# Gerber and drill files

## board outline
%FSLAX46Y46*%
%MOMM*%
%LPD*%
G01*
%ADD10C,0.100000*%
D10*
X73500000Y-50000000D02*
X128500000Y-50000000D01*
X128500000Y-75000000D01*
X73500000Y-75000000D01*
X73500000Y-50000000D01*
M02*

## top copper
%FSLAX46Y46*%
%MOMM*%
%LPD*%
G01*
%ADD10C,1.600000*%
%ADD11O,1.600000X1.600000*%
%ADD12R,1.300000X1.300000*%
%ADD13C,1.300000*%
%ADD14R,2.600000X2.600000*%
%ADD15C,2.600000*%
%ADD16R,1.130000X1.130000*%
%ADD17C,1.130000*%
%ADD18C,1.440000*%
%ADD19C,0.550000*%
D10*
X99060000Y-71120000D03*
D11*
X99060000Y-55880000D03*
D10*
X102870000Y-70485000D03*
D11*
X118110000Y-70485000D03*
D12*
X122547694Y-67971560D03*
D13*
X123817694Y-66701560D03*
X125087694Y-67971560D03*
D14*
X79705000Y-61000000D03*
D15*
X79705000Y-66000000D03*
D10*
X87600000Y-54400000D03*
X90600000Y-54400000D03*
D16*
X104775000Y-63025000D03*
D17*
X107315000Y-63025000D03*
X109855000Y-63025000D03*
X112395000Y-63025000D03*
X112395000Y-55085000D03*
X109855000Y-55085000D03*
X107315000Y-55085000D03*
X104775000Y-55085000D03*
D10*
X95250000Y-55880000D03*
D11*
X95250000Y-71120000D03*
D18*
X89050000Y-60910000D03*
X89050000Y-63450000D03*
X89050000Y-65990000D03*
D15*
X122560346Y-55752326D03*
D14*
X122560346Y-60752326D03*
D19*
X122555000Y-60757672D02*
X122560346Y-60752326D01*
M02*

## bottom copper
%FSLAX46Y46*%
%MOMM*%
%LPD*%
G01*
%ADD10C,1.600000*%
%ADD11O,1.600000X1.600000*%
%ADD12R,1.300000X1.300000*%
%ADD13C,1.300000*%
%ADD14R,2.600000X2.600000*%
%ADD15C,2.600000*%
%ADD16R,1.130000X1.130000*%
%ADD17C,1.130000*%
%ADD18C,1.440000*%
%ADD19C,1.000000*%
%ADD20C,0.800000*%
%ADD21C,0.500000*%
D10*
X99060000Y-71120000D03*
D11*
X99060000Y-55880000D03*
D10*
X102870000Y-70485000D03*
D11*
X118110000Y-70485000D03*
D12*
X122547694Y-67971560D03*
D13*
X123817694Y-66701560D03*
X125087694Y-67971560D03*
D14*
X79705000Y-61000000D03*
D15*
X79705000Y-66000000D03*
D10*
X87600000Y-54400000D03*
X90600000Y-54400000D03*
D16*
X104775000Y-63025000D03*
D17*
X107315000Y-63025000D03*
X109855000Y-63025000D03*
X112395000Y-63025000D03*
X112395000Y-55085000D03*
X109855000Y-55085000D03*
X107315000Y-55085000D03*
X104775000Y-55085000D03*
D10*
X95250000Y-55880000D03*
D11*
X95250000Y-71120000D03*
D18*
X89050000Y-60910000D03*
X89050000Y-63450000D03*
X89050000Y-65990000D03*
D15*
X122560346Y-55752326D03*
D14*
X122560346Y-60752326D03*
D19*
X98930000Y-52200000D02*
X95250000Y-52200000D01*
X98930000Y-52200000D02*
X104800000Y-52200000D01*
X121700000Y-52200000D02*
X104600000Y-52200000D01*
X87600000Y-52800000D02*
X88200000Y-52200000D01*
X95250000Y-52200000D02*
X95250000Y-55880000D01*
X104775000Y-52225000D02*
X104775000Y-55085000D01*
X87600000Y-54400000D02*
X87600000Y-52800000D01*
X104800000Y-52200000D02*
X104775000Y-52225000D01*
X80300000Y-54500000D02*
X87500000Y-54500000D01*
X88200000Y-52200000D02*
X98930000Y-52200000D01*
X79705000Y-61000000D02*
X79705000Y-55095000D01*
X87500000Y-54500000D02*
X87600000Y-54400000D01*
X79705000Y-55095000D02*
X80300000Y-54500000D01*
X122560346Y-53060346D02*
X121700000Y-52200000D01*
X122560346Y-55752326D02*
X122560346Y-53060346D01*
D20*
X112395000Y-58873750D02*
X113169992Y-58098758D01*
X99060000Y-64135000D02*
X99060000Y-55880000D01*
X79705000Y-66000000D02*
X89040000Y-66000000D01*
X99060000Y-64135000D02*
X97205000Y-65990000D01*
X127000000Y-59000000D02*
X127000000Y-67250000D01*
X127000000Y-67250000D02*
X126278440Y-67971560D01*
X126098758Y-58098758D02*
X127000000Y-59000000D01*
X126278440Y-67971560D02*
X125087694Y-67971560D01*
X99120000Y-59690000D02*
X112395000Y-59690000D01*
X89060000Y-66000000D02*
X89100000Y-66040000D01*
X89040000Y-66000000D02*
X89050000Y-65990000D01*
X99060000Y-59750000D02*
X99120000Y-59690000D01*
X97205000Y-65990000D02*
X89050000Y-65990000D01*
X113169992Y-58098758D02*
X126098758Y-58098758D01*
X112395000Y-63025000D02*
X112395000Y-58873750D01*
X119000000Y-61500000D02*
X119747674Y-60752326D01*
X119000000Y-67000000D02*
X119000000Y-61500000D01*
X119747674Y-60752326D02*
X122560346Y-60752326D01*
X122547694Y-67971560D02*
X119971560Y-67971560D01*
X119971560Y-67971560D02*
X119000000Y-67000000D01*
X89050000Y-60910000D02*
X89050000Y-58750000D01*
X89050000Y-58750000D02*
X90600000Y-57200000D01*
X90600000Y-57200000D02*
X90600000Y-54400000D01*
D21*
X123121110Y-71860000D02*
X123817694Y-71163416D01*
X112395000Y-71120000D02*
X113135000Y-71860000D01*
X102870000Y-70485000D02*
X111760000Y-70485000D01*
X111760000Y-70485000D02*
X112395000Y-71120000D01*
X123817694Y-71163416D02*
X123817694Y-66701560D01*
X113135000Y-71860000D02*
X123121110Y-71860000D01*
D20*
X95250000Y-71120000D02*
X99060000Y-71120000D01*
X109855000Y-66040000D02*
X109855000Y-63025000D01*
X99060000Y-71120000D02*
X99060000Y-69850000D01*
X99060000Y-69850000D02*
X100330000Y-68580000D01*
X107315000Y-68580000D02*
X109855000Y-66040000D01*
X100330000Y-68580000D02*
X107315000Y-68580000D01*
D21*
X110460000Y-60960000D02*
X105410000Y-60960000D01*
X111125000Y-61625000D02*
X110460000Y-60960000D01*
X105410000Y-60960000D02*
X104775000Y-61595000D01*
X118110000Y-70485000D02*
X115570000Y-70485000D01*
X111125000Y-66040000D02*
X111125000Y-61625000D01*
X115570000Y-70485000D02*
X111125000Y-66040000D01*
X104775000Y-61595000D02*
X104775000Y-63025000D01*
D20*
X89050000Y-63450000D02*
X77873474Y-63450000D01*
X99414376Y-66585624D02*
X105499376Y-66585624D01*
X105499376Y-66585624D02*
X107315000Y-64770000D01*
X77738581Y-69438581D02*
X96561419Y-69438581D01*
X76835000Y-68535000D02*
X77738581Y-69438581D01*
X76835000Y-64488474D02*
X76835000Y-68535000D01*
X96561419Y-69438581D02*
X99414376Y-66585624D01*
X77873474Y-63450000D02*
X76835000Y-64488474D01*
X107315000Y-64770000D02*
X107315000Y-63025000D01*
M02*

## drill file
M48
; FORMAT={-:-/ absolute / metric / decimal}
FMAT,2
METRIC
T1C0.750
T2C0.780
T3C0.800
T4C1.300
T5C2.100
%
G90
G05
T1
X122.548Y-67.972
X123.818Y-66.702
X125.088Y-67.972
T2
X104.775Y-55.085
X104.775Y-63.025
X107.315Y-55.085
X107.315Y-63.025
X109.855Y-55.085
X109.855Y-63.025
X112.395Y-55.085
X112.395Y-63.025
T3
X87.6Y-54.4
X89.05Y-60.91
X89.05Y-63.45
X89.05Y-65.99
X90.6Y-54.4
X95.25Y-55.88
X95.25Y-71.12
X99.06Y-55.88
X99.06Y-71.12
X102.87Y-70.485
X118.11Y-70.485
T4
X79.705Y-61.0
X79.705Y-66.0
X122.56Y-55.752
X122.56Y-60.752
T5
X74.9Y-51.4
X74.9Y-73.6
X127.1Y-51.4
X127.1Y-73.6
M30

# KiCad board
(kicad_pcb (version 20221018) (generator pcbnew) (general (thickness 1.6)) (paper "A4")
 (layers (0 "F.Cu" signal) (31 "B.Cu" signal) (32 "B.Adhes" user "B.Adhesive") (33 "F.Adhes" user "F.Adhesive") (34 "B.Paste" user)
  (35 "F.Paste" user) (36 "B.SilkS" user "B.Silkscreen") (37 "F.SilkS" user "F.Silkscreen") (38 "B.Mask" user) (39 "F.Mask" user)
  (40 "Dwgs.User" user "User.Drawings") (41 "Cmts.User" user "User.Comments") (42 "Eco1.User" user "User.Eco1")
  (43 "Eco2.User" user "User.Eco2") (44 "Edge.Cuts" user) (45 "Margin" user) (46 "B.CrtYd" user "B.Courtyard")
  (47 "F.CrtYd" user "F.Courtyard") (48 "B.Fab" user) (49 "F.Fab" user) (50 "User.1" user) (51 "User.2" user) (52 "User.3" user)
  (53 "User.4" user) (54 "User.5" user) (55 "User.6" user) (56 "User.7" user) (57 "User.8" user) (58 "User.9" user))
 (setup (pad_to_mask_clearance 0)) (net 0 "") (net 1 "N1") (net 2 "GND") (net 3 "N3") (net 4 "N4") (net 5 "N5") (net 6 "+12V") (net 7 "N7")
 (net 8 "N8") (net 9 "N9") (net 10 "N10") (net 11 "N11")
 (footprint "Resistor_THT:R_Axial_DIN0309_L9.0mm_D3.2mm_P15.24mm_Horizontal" (layer "F.Cu") (at 99.06 71.12 90)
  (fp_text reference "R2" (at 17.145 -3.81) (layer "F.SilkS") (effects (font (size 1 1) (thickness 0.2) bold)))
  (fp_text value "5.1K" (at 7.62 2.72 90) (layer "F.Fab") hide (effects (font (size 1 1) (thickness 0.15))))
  (pad "1" thru_hole circle (at 0 0 90) (size 1.6 1.6) (drill 0.8) (layers "*.Cu" "*.Mask") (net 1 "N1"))
  (pad "2" thru_hole oval (at 15.24 0 90) (size 1.6 1.6) (drill 0.8) (layers "*.Cu" "*.Mask") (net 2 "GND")))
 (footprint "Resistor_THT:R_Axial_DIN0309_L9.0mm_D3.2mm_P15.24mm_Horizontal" (layer "F.Cu") (at 102.87 70.485)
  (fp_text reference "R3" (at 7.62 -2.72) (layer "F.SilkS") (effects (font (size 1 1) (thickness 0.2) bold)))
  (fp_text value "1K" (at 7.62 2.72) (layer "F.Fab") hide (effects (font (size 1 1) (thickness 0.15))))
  (pad "1" thru_hole circle (at 0 0) (size 1.6 1.6) (drill 0.8) (layers "*.Cu" "*.Mask") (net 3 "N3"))
  (pad "2" thru_hole oval (at 15.24 0) (size 1.6 1.6) (drill 0.8) (layers "*.Cu" "*.Mask") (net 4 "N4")))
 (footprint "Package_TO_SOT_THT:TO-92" (layer "F.Cu") (at 122.547694 67.97156)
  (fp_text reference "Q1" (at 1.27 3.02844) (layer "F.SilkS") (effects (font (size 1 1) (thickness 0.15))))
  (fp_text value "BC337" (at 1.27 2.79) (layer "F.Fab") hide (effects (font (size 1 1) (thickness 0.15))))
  (pad "1" thru_hole rect (at 0 0) (size 1.3 1.3) (drill 0.75) (layers "*.Cu" "*.Mask") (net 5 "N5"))
  (pad "2" thru_hole circle (at 1.27 -1.27) (size 1.3 1.3) (drill 0.75) (layers "*.Cu" "*.Mask") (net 3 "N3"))
  (pad "3" thru_hole circle (at 2.54 0) (size 1.3 1.3) (drill 0.75) (layers "*.Cu" "*.Mask") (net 2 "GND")))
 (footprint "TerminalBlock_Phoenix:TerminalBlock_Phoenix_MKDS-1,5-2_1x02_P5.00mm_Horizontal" (layer "F.Cu") (at 79.705 61 -90)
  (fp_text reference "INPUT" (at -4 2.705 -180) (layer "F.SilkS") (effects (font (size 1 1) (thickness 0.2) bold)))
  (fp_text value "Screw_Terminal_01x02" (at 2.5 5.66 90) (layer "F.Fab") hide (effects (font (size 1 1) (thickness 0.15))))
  (pad "1" thru_hole rect (at 0 0 270) (size 2.6 2.6) (drill 1.3) (layers "*.Cu" "*.Mask") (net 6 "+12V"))
  (pad "2" thru_hole circle (at 5 0 270) (size 2.6 2.6) (drill 1.3) (layers "*.Cu" "*.Mask") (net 2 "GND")))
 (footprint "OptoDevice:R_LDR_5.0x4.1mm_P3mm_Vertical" (layer "F.Cu") (at 87.6 54.4)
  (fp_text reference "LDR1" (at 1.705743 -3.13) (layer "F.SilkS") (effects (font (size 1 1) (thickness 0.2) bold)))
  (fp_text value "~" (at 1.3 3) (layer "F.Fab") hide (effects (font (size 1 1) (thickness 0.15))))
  (pad "1" thru_hole circle (at 0 0) (size 1.6 1.6) (drill 0.8) (layers "*.Cu" "*.Mask") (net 6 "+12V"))
  (pad "2" thru_hole circle (at 3 0) (size 1.6 1.6) (drill 0.8) (layers "*.Cu" "*.Mask") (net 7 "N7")))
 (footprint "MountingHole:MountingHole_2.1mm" (layer "F.Cu") (at 74.9 51.4)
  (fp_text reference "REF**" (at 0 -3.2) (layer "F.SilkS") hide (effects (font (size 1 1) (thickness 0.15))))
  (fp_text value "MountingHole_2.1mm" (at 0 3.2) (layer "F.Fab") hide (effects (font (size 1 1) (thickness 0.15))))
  (pad "" np_thru_hole circle (at 0 0) (size 2.1 2.1) (drill 2.1) (layers "F&B.Cu" "*.Mask")))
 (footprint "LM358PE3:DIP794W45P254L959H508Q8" (layer "F.Cu") (at 108.585 59.055 90)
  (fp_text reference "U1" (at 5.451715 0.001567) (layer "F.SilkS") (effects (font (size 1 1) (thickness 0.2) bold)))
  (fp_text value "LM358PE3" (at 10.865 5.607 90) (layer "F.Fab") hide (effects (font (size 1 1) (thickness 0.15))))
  (pad "1" thru_hole rect (at -3.97 -3.81 90) (size 1.13 1.13) (drill 0.78) (layers "*.Cu" "*.Mask") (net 4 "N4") (solder_mask_margin 0.102))
  (pad "2" thru_hole circle (at -3.97 -1.27 90) (size 1.13 1.13) (drill 0.78) (layers "*.Cu" "*.Mask") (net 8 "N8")
   (solder_mask_margin 0.102))
  (pad "3" thru_hole circle (at -3.97 1.27 90) (size 1.13 1.13) (drill 0.78) (layers "*.Cu" "*.Mask") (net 1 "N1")
   (solder_mask_margin 0.102))
  (pad "4" thru_hole circle (at -3.97 3.81 90) (size 1.13 1.13) (drill 0.78) (layers "*.Cu" "*.Mask") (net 2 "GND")
   (solder_mask_margin 0.102))
  (pad "5" thru_hole circle (at 3.97 3.81 90) (size 1.13 1.13) (drill 0.78) (layers "*.Cu" "*.Mask") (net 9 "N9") (solder_mask_margin 0.102))
  (pad "6" thru_hole circle (at 3.97 1.27 90) (size 1.13 1.13) (drill 0.78) (layers "*.Cu" "*.Mask") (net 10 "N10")
   (solder_mask_margin 0.102))
  (pad "7" thru_hole circle (at 3.97 -1.27 90) (size 1.13 1.13) (drill 0.78) (layers "*.Cu" "*.Mask") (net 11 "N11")
   (solder_mask_margin 0.102))
  (pad "8" thru_hole circle (at 3.97 -3.81 90) (size 1.13 1.13) (drill 0.78) (layers "*.Cu" "*.Mask") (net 6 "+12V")
   (solder_mask_margin 0.102)))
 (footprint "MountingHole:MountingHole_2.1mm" (layer "F.Cu") (at 74.9 73.6)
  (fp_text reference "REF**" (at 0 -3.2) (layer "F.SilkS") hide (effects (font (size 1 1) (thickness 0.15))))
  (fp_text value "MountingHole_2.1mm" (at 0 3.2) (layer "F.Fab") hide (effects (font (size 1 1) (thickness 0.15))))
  (pad "" np_thru_hole circle (at 0 0) (size 2.1 2.1) (drill 2.1) (layers "F&B.Cu" "*.Mask")))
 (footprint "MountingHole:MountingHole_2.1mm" (layer "F.Cu") (at 127.1 51.4)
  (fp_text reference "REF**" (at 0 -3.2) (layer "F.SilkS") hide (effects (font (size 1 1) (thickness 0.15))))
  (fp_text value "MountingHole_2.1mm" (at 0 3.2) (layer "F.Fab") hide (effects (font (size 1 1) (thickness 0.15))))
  (pad "" np_thru_hole circle (at 0 0) (size 2.1 2.1) (drill 2.1) (layers "F&B.Cu" "*.Mask")))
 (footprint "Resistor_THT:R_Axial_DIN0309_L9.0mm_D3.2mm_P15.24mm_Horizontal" (layer "F.Cu") (at 95.25 55.88 -90)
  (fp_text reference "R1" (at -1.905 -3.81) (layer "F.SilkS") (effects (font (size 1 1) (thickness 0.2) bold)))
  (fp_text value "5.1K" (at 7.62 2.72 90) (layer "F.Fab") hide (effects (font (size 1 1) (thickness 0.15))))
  (pad "1" thru_hole circle (at 0 0 270) (size 1.6 1.6) (drill 0.8) (layers "*.Cu" "*.Mask") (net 6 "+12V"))
  (pad "2" thru_hole oval (at 15.24 0 270) (size 1.6 1.6) (drill 0.8) (layers "*.Cu" "*.Mask") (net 1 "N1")))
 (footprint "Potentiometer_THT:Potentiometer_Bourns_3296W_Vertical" (layer "F.Cu") (at 89.05 60.91 90)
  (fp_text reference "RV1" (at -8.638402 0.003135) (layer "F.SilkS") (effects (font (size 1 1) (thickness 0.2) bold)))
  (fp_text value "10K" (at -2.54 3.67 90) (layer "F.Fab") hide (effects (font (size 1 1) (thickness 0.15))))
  (pad "1" thru_hole circle (at 0 0 90) (size 1.44 1.44) (drill 0.8) (layers "*.Cu" "*.Mask") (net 7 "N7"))
  (pad "2" thru_hole circle (at -2.54 0 90) (size 1.44 1.44) (drill 0.8) (layers "*.Cu" "*.Mask") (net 8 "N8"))
  (pad "3" thru_hole circle (at -5.08 0 90) (size 1.44 1.44) (drill 0.8) (layers "*.Cu" "*.Mask") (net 2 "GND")))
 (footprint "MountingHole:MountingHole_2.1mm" (layer "F.Cu") (at 127.1 73.6)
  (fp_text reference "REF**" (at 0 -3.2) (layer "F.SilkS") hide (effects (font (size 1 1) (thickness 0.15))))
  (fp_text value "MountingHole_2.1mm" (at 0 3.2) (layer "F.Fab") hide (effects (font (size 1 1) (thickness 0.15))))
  (pad "" np_thru_hole circle (at 0 0) (size 2.1 2.1) (drill 2.1) (layers "*.Cu" "*.Mask")))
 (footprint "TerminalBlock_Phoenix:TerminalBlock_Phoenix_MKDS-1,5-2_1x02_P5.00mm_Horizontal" (layer "F.Cu") (at 122.560346 60.752326 90)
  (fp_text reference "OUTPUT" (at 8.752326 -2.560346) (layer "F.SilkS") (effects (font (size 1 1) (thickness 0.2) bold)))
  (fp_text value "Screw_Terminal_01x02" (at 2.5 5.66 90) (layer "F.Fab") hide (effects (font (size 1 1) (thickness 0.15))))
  (pad "1" thru_hole circle (at 5 0 90) (size 2.6 2.6) (drill 1.3) (layers "*.Cu" "*.Mask") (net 6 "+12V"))
  (pad "2" thru_hole rect (at 0 0 90) (size 2.6 2.6) (drill 1.3) (layers "*.Cu" "*.Mask") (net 5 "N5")))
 (gr_rect (start 73.5 50) (end 128.5 75) (stroke (width 0.1) (type default)) (fill none) (layer "Edge.Cuts"))
 (segment (start 98.93 52.2) (end 95.25 52.2) (width 1) (layer "B.Cu") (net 6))
 (segment (start 98.93 52.2) (end 104.8 52.2) (width 1) (layer "B.Cu") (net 6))
 (segment (start 121.7 52.2) (end 104.6 52.2) (width 1) (layer "B.Cu") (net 6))
 (segment (start 87.6 52.8) (end 88.2 52.2) (width 1) (layer "B.Cu") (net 6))
 (segment (start 95.25 52.2) (end 95.25 55.88) (width 1) (layer "B.Cu") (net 6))
 (segment (start 104.775 52.225) (end 104.775 55.085) (width 1) (layer "B.Cu") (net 6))
 (segment (start 87.6 54.4) (end 87.6 52.8) (width 1) (layer "B.Cu") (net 6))
 (segment (start 104.8 52.2) (end 104.775 52.225) (width 1) (layer "B.Cu") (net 6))
 (segment (start 80.3 54.5) (end 87.5 54.5) (width 1) (layer "B.Cu") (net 6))
 (segment (start 88.2 52.2) (end 98.93 52.2) (width 1) (layer "B.Cu") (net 6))
 (segment (start 79.705 61) (end 79.705 55.095) (width 1) (layer "B.Cu") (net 6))
 (segment (start 87.5 54.5) (end 87.6 54.4) (width 1) (layer "B.Cu") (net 6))
 (segment (start 79.705 55.095) (end 80.3 54.5) (width 1) (layer "B.Cu") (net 6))
 (segment (start 122.560346 53.060346) (end 121.7 52.2) (width 1) (layer "B.Cu") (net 6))
 (segment (start 122.560346 55.752326) (end 122.560346 53.060346) (width 1) (layer "B.Cu") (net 6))
 (segment (start 112.395 58.87375) (end 113.169992 58.098758) (width 0.8) (layer "B.Cu") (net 2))
 (segment (start 99.06 64.135) (end 99.06 55.88) (width 0.8) (layer "B.Cu") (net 2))
 (segment (start 79.705 66) (end 89.04 66) (width 0.8) (layer "B.Cu") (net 2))
 (segment (start 99.06 64.135) (end 97.205 65.99) (width 0.8) (layer "B.Cu") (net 2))
 (segment (start 127 59) (end 127 67.25) (width 0.8) (layer "B.Cu") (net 2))
 (segment (start 127 67.25) (end 126.27844 67.97156) (width 0.8) (layer "B.Cu") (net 2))
 (segment (start 126.098758 58.098758) (end 127 59) (width 0.8) (layer "B.Cu") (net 2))
 (segment (start 126.27844 67.97156) (end 125.087694 67.97156) (width 0.8) (layer "B.Cu") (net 2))
 (segment (start 99.12 59.69) (end 112.395 59.69) (width 0.8) (layer "B.Cu") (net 2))
 (segment (start 89.06 66) (end 89.1 66.04) (width 0.8) (layer "B.Cu") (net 2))
 (segment (start 89.04 66) (end 89.05 65.99) (width 0.8) (layer "B.Cu") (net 2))
 (segment (start 99.06 59.75) (end 99.12 59.69) (width 0.8) (layer "B.Cu") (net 2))
 (segment (start 97.205 65.99) (end 89.05 65.99) (width 0.8) (layer "B.Cu") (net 2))
 (segment (start 113.169992 58.098758) (end 126.098758 58.098758) (width 0.8) (layer "B.Cu") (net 2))
 (segment (start 112.395 63.025) (end 112.395 58.87375) (width 0.8) (layer "B.Cu") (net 2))
 (segment (start 122.555 60.757672) (end 122.560346 60.752326) (width 0.55) (layer "F.Cu") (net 5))
 (segment (start 119 61.5) (end 119.747674 60.752326) (width 0.8) (layer "B.Cu") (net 5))
 (segment (start 119 67) (end 119 61.5) (width 0.8) (layer "B.Cu") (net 5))
 (segment (start 119.747674 60.752326) (end 122.560346 60.752326) (width 0.8) (layer "B.Cu") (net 5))
 (segment (start 122.547694 67.97156) (end 119.97156 67.97156) (width 0.8) (layer "B.Cu") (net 5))
 (segment (start 119.97156 67.97156) (end 119 67) (width 0.8) (layer "B.Cu") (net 5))
 (segment (start 89.05 60.91) (end 89.05 58.75) (width 0.8) (layer "B.Cu") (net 7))
 (segment (start 89.05 58.75) (end 90.6 57.2) (width 0.8) (layer "B.Cu") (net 7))
 (segment (start 90.6 57.2) (end 90.6 54.4) (width 0.8) (layer "B.Cu") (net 7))
 (segment (start 123.12111 71.86) (end 123.817694 71.163416) (width 0.5) (layer "B.Cu") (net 3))
 (segment (start 112.395 71.12) (end 113.135 71.86) (width 0.5) (layer "B.Cu") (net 3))
 (segment (start 102.87 70.485) (end 111.76 70.485) (width 0.5) (layer "B.Cu") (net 3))
 (segment (start 111.76 70.485) (end 112.395 71.12) (width 0.5) (layer "B.Cu") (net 3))
 (segment (start 123.817694 71.163416) (end 123.817694 66.70156) (width 0.5) (layer "B.Cu") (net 3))
 (segment (start 113.135 71.86) (end 123.12111 71.86) (width 0.5) (layer "B.Cu") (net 3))
 (segment (start 95.25 71.12) (end 99.06 71.12) (width 0.8) (layer "B.Cu") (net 1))
 (segment (start 109.855 66.04) (end 109.855 63.025) (width 0.8) (layer "B.Cu") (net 1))
 (segment (start 99.06 71.12) (end 99.06 69.85) (width 0.8) (layer "B.Cu") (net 1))
 (segment (start 99.06 69.85) (end 100.33 68.58) (width 0.8) (layer "B.Cu") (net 1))
 (segment (start 107.315 68.58) (end 109.855 66.04) (width 0.8) (layer "B.Cu") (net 1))
 (segment (start 100.33 68.58) (end 107.315 68.58) (width 0.8) (layer "B.Cu") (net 1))
 (segment (start 110.46 60.96) (end 105.41 60.96) (width 0.5) (layer "B.Cu") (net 4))
 (segment (start 111.125 61.625) (end 110.46 60.96) (width 0.5) (layer "B.Cu") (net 4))
 (segment (start 105.41 60.96) (end 104.775 61.595) (width 0.5) (layer "B.Cu") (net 4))
 (segment (start 118.11 70.485) (end 115.57 70.485) (width 0.5) (layer "B.Cu") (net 4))
 (segment (start 111.125 66.04) (end 111.125 61.625) (width 0.5) (layer "B.Cu") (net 4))
 (segment (start 115.57 70.485) (end 111.125 66.04) (width 0.5) (layer "B.Cu") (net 4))
 (segment (start 104.775 61.595) (end 104.775 63.025) (width 0.5) (layer "B.Cu") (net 4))
 (segment (start 89.05 63.45) (end 77.873474 63.45) (width 0.8) (layer "B.Cu") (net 8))
 (segment (start 99.414376 66.585624) (end 105.499376 66.585624) (width 0.8) (layer "B.Cu") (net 8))
 (segment (start 105.499376 66.585624) (end 107.315 64.77) (width 0.8) (layer "B.Cu") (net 8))
 (segment (start 77.738581 69.438581) (end 96.561419 69.438581) (width 0.8) (layer "B.Cu") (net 8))
 (segment (start 76.835 68.535) (end 77.738581 69.438581) (width 0.8) (layer "B.Cu") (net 8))
 (segment (start 76.835 64.488474) (end 76.835 68.535) (width 0.8) (layer "B.Cu") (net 8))
 (segment (start 96.561419 69.438581) (end 99.414376 66.585624) (width 0.8) (layer "B.Cu") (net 8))
 (segment (start 77.873474 63.45) (end 76.835 64.488474) (width 0.8) (layer "B.Cu") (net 8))
 (segment (start 107.315 64.77) (end 107.315 63.025) (width 0.8) (layer "B.Cu") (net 8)))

